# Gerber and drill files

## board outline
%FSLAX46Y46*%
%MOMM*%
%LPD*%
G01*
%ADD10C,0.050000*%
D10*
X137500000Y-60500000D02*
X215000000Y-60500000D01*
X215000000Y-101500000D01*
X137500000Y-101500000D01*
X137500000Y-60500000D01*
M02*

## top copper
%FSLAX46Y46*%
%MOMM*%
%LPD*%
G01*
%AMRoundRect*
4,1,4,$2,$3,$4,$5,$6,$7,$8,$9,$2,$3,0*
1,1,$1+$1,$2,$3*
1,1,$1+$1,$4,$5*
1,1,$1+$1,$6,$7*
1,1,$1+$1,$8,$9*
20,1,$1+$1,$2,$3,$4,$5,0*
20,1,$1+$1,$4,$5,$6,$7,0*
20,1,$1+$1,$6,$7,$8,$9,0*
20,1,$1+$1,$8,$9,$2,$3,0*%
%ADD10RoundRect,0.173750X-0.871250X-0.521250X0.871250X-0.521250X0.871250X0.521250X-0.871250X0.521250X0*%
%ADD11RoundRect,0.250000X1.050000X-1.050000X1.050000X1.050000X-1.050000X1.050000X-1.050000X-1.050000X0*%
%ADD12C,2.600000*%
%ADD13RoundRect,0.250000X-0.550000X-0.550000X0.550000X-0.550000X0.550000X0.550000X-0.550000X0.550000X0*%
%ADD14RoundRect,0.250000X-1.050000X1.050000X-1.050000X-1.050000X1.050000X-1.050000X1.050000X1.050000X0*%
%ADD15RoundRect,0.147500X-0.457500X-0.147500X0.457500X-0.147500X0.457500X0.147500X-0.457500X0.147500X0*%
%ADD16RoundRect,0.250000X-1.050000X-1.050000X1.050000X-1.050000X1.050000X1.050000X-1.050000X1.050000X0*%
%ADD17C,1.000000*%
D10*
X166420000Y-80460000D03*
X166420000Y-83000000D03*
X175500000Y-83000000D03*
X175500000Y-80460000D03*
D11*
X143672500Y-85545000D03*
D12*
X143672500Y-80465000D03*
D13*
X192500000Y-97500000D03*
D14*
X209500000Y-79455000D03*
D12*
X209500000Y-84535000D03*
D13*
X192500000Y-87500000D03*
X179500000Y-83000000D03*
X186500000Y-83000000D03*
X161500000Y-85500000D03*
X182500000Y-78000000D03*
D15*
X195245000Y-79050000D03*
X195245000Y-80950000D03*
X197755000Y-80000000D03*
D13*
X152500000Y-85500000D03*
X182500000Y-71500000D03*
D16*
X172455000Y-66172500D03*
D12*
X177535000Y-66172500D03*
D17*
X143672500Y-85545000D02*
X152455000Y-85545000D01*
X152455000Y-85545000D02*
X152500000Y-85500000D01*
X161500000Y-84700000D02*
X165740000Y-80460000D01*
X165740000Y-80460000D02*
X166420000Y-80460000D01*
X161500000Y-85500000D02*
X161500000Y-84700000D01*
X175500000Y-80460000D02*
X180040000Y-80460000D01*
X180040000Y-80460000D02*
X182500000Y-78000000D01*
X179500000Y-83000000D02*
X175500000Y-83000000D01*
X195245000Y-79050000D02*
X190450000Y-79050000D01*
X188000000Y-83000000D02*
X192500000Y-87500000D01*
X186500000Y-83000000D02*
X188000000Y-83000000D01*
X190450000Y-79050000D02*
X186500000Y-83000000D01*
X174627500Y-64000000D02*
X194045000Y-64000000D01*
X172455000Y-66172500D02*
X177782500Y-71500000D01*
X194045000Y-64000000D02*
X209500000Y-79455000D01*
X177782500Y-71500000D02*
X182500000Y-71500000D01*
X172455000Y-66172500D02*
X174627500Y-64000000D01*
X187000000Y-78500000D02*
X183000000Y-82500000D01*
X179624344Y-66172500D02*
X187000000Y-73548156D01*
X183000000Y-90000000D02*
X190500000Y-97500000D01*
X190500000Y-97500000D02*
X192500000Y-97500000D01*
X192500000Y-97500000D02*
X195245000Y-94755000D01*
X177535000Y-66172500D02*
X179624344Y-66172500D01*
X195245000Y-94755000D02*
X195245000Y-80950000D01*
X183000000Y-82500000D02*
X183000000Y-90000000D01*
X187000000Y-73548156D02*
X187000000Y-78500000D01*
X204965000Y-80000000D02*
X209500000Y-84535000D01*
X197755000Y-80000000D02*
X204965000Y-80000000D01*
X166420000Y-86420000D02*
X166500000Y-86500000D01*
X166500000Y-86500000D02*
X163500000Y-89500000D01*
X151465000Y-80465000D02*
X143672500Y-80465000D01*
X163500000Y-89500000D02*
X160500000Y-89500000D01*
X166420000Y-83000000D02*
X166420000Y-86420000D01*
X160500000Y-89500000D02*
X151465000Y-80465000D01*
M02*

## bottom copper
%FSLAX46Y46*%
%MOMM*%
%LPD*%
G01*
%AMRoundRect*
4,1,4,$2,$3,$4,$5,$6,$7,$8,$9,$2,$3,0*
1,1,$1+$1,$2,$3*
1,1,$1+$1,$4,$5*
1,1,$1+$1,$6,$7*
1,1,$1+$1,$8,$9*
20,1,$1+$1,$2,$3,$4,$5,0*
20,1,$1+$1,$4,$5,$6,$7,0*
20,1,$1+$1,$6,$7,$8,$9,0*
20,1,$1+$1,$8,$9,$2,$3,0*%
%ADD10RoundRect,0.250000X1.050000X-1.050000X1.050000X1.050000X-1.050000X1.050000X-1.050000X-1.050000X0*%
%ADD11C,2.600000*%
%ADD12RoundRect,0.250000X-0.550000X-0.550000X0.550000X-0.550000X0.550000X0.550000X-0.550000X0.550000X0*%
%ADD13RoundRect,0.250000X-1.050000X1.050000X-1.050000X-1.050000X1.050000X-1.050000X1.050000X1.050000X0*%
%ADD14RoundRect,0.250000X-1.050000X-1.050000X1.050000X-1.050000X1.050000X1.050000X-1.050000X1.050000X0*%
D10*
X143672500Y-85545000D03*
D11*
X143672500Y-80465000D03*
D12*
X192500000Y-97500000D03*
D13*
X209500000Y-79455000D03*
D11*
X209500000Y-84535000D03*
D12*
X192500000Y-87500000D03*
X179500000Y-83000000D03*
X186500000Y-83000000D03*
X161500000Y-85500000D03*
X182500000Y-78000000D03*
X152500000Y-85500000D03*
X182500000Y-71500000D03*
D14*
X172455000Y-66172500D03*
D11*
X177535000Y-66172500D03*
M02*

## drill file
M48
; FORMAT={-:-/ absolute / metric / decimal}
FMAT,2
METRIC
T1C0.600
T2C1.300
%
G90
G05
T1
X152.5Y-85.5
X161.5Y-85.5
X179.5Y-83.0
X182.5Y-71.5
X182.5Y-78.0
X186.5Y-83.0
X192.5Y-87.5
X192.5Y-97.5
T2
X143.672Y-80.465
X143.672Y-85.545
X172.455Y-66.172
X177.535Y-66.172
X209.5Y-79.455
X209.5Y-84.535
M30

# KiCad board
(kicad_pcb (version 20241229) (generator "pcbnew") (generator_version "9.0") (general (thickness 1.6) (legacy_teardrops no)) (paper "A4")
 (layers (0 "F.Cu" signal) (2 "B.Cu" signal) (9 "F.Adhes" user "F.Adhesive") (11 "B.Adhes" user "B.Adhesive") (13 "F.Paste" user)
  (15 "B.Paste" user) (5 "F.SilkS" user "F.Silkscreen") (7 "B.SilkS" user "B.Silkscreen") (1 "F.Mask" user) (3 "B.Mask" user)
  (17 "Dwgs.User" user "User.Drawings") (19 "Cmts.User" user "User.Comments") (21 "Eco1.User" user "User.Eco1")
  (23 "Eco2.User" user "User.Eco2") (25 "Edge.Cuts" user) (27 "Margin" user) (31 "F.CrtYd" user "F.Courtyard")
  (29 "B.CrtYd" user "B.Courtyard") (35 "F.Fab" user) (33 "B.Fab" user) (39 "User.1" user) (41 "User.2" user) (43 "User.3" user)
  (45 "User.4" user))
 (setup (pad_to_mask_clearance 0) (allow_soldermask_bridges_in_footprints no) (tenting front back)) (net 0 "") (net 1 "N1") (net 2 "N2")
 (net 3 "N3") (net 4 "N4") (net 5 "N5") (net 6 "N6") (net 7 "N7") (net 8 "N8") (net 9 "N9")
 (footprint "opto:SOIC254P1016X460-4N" (layer "F.Cu") (at 170.96 81.73)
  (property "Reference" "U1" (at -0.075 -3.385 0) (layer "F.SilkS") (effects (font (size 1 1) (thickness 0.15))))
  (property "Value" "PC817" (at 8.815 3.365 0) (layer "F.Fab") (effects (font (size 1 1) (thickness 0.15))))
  (pad "1" smd roundrect (at -4.54 -1.27) (size 2.09 1.39) (layers "F.Cu" "F.Mask" "F.Paste") (roundrect_rratio 0.125) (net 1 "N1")
   (solder_mask_margin 0.102))
  (pad "2" smd roundrect (at -4.54 1.27) (size 2.09 1.39) (layers "F.Cu" "F.Mask" "F.Paste") (roundrect_rratio 0.125) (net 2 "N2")
   (solder_mask_margin 0.102))
  (pad "3" smd roundrect (at 4.54 1.27) (size 2.09 1.39) (layers "F.Cu" "F.Mask" "F.Paste") (roundrect_rratio 0.125) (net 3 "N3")
   (solder_mask_margin 0.102))
  (pad "4" smd roundrect (at 4.54 -1.27) (size 2.09 1.39) (layers "F.Cu" "F.Mask" "F.Paste") (roundrect_rratio 0.125) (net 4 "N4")
   (solder_mask_margin 0.102)))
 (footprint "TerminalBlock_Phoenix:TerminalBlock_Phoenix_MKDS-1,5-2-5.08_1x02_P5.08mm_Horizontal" (layer "F.Cu") (at 143.6725 85.545 90)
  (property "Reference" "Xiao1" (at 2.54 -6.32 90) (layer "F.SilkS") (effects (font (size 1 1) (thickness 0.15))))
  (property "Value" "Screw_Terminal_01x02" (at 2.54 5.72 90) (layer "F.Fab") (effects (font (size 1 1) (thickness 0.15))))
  (pad "1" thru_hole roundrect (at 0 0 90) (size 2.6 2.6) (drill 1.3) (layers "*.Cu" "*.Mask") (remove_unused_layers no)
   (roundrect_rratio 0.096154) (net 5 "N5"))
  (pad "2" thru_hole circle (at 5.08 0 90) (size 2.6 2.6) (drill 1.3) (layers "*.Cu" "*.Mask") (remove_unused_layers no) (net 2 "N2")))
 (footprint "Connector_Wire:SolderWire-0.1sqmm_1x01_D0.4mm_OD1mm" (layer "F.Cu") (at 192.5 97.5)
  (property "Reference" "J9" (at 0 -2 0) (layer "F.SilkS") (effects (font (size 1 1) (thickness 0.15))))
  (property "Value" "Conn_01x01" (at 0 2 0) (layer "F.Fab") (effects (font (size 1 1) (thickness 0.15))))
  (pad "1" thru_hole roundrect (at 0 0) (size 1.6 1.6) (drill 0.6) (layers "*.Cu" "*.Mask") (remove_unused_layers no)
   (roundrect_rratio 0.15625) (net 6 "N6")))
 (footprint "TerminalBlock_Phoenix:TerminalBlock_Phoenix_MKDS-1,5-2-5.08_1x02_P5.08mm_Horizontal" (layer "F.Cu") (at 209.5 79.455 -90)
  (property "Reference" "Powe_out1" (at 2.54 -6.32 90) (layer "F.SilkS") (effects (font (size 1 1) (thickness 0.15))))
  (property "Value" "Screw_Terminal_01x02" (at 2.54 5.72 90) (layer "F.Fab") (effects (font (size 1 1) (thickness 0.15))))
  (pad "1" thru_hole roundrect (at 0 0 270) (size 2.6 2.6) (drill 1.3) (layers "*.Cu" "*.Mask") (remove_unused_layers no)
   (roundrect_rratio 0.096154) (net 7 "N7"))
  (pad "2" thru_hole circle (at 5.08 0 270) (size 2.6 2.6) (drill 1.3) (layers "*.Cu" "*.Mask") (remove_unused_layers no) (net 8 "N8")))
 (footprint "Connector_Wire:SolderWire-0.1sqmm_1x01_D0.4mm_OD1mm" (layer "F.Cu") (at 192.5 87.5)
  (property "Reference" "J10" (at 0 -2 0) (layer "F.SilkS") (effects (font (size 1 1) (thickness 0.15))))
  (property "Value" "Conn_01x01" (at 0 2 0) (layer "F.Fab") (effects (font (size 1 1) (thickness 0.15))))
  (pad "1" thru_hole roundrect (at 0 0) (size 1.6 1.6) (drill 0.6) (layers "*.Cu" "*.Mask") (remove_unused_layers no)
   (roundrect_rratio 0.15625) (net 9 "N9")))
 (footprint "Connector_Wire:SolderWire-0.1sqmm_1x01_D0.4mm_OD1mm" (layer "F.Cu") (at 179.5 83)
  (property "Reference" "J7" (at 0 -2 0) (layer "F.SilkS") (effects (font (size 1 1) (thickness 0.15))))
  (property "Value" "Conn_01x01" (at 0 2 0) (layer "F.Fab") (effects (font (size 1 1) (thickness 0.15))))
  (pad "1" thru_hole roundrect (at 0 0) (size 1.6 1.6) (drill 0.6) (layers "*.Cu" "*.Mask") (remove_unused_layers no)
   (roundrect_rratio 0.15625) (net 3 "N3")))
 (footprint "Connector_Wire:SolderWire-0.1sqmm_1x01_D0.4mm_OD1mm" (layer "F.Cu") (at 186.5 83)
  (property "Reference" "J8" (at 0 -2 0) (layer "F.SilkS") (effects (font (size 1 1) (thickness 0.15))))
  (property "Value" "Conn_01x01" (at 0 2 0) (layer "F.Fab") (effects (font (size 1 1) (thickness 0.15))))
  (pad "1" thru_hole roundrect (at 0 0) (size 1.6 1.6) (drill 0.6) (layers "*.Cu" "*.Mask") (remove_unused_layers no)
   (roundrect_rratio 0.15625) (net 9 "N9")))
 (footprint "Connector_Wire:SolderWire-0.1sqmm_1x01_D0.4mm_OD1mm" (layer "F.Cu") (at 161.5 85.5)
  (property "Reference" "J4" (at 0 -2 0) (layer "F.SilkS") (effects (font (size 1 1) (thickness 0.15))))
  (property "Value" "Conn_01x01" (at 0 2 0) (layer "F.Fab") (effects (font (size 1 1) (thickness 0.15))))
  (pad "1" thru_hole roundrect (at 0 0) (size 1.6 1.6) (drill 0.6) (layers "*.Cu" "*.Mask") (remove_unused_layers no)
   (roundrect_rratio 0.15625) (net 1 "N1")))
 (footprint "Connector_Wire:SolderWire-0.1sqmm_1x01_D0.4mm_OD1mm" (layer "F.Cu") (at 182.5 78)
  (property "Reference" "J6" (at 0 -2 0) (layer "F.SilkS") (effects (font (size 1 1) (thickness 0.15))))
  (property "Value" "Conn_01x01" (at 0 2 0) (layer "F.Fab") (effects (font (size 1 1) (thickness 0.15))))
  (pad "1" thru_hole roundrect (at 0 0) (size 1.6 1.6) (drill 0.6) (layers "*.Cu" "*.Mask") (remove_unused_layers no)
   (roundrect_rratio 0.15625) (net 4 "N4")))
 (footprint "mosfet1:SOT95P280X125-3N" (layer "F.Cu") (at 196.5 80)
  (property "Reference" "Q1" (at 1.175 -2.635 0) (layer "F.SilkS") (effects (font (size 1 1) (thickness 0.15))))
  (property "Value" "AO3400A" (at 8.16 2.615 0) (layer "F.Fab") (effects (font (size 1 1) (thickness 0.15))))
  (pad "1" smd roundrect (at -1.255 -0.95) (size 1.21 0.59) (layers "F.Cu" "F.Mask" "F.Paste") (roundrect_rratio 0.25) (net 9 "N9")
   (solder_mask_margin 0.102))
  (pad "2" smd roundrect (at -1.255 0.95) (size 1.21 0.59) (layers "F.Cu" "F.Mask" "F.Paste") (roundrect_rratio 0.25) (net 6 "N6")
   (solder_mask_margin 0.102))
  (pad "3" smd roundrect (at 1.255 0) (size 1.21 0.59) (layers "F.Cu" "F.Mask" "F.Paste") (roundrect_rratio 0.25) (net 8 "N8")
   (solder_mask_margin 0.102)))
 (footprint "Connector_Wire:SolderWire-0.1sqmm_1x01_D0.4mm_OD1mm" (layer "F.Cu") (at 152.5 85.5)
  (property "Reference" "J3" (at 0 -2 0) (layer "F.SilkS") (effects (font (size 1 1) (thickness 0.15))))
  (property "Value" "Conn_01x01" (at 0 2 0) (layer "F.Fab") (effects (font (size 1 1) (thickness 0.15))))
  (pad "1" thru_hole roundrect (at 0 0) (size 1.6 1.6) (drill 0.6) (layers "*.Cu" "*.Mask") (remove_unused_layers no)
   (roundrect_rratio 0.15625) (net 5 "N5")))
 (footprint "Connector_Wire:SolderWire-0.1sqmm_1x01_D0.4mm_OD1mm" (layer "F.Cu") (at 182.5 71.5)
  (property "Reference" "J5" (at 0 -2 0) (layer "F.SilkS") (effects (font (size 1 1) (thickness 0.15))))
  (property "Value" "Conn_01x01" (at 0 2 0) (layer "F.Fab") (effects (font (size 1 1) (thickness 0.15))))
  (pad "1" thru_hole roundrect (at 0 0) (size 1.6 1.6) (drill 0.6) (layers "*.Cu" "*.Mask") (remove_unused_layers no)
   (roundrect_rratio 0.15625) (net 7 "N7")))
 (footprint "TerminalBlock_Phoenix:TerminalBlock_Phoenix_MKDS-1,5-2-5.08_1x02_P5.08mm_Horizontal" (layer "F.Cu") (at 172.455 66.1725)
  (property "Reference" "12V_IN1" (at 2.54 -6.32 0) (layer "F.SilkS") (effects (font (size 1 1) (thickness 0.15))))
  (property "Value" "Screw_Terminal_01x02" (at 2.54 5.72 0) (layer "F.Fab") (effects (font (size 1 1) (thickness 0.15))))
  (pad "1" thru_hole roundrect (at 0 0) (size 2.6 2.6) (drill 1.3) (layers "*.Cu" "*.Mask") (remove_unused_layers no)
   (roundrect_rratio 0.096154) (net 7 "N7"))
  (pad "2" thru_hole circle (at 5.08 0) (size 2.6 2.6) (drill 1.3) (layers "*.Cu" "*.Mask") (remove_unused_layers no) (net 6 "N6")))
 (gr_rect (start 137.5 60.5) (end 215 101.5) (stroke (width 0.05) (type default)) (fill no) (layer "Edge.Cuts"))
 (segment (start 143.6725 85.545) (end 152.455 85.545) (width 1) (layer "F.Cu") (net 5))
 (segment (start 152.455 85.545) (end 152.5 85.5) (width 1) (layer "F.Cu") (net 5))
 (segment (start 161.5 84.7) (end 165.74 80.46) (width 1) (layer "F.Cu") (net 1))
 (segment (start 165.74 80.46) (end 166.42 80.46) (width 1) (layer "F.Cu") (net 1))
 (segment (start 161.5 85.5) (end 161.5 84.7) (width 1) (layer "F.Cu") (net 1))
 (segment (start 175.5 80.46) (end 180.04 80.46) (width 1) (layer "F.Cu") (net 4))
 (segment (start 180.04 80.46) (end 182.5 78) (width 1) (layer "F.Cu") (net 4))
 (segment (start 179.5 83) (end 175.5 83) (width 1) (layer "F.Cu") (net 3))
 (segment (start 195.245 79.05) (end 190.45 79.05) (width 1) (layer "F.Cu") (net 9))
 (segment (start 188 83) (end 192.5 87.5) (width 1) (layer "F.Cu") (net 9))
 (segment (start 186.5 83) (end 188 83) (width 1) (layer "F.Cu") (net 9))
 (segment (start 190.45 79.05) (end 186.5 83) (width 1) (layer "F.Cu") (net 9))
 (segment (start 174.6275 64) (end 194.045 64) (width 1) (layer "F.Cu") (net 7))
 (segment (start 172.455 66.1725) (end 177.7825 71.5) (width 1) (layer "F.Cu") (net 7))
 (segment (start 194.045 64) (end 209.5 79.455) (width 1) (layer "F.Cu") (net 7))
 (segment (start 177.7825 71.5) (end 182.5 71.5) (width 1) (layer "F.Cu") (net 7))
 (segment (start 172.455 66.1725) (end 174.6275 64) (width 1) (layer "F.Cu") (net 7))
 (segment (start 187 78.5) (end 183 82.5) (width 1) (layer "F.Cu") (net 6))
 (segment (start 179.624344 66.1725) (end 187 73.548156) (width 1) (layer "F.Cu") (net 6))
 (segment (start 183 90) (end 190.5 97.5) (width 1) (layer "F.Cu") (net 6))
 (segment (start 190.5 97.5) (end 192.5 97.5) (width 1) (layer "F.Cu") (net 6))
 (segment (start 192.5 97.5) (end 195.245 94.755) (width 1) (layer "F.Cu") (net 6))
 (segment (start 177.535 66.1725) (end 179.624344 66.1725) (width 1) (layer "F.Cu") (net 6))
 (segment (start 195.245 94.755) (end 195.245 80.95) (width 1) (layer "F.Cu") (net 6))
 (segment (start 183 82.5) (end 183 90) (width 1) (layer "F.Cu") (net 6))
 (segment (start 187 73.548156) (end 187 78.5) (width 1) (layer "F.Cu") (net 6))
 (segment (start 204.965 80) (end 209.5 84.535) (width 1) (layer "F.Cu") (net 8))
 (segment (start 197.755 80) (end 204.965 80) (width 1) (layer "F.Cu") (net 8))
 (segment (start 166.42 86.42) (end 166.5 86.5) (width 1) (layer "F.Cu") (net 2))
 (segment (start 166.5 86.5) (end 163.5 89.5) (width 1) (layer "F.Cu") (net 2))
 (segment (start 151.465 80.465) (end 143.6725 80.465) (width 1) (layer "F.Cu") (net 2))
 (segment (start 163.5 89.5) (end 160.5 89.5) (width 1) (layer "F.Cu") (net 2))
 (segment (start 166.42 83) (end 166.42 86.42) (width 1) (layer "F.Cu") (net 2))
 (segment (start 160.5 89.5) (end 151.465 80.465) (width 1) (layer "F.Cu") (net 2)))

